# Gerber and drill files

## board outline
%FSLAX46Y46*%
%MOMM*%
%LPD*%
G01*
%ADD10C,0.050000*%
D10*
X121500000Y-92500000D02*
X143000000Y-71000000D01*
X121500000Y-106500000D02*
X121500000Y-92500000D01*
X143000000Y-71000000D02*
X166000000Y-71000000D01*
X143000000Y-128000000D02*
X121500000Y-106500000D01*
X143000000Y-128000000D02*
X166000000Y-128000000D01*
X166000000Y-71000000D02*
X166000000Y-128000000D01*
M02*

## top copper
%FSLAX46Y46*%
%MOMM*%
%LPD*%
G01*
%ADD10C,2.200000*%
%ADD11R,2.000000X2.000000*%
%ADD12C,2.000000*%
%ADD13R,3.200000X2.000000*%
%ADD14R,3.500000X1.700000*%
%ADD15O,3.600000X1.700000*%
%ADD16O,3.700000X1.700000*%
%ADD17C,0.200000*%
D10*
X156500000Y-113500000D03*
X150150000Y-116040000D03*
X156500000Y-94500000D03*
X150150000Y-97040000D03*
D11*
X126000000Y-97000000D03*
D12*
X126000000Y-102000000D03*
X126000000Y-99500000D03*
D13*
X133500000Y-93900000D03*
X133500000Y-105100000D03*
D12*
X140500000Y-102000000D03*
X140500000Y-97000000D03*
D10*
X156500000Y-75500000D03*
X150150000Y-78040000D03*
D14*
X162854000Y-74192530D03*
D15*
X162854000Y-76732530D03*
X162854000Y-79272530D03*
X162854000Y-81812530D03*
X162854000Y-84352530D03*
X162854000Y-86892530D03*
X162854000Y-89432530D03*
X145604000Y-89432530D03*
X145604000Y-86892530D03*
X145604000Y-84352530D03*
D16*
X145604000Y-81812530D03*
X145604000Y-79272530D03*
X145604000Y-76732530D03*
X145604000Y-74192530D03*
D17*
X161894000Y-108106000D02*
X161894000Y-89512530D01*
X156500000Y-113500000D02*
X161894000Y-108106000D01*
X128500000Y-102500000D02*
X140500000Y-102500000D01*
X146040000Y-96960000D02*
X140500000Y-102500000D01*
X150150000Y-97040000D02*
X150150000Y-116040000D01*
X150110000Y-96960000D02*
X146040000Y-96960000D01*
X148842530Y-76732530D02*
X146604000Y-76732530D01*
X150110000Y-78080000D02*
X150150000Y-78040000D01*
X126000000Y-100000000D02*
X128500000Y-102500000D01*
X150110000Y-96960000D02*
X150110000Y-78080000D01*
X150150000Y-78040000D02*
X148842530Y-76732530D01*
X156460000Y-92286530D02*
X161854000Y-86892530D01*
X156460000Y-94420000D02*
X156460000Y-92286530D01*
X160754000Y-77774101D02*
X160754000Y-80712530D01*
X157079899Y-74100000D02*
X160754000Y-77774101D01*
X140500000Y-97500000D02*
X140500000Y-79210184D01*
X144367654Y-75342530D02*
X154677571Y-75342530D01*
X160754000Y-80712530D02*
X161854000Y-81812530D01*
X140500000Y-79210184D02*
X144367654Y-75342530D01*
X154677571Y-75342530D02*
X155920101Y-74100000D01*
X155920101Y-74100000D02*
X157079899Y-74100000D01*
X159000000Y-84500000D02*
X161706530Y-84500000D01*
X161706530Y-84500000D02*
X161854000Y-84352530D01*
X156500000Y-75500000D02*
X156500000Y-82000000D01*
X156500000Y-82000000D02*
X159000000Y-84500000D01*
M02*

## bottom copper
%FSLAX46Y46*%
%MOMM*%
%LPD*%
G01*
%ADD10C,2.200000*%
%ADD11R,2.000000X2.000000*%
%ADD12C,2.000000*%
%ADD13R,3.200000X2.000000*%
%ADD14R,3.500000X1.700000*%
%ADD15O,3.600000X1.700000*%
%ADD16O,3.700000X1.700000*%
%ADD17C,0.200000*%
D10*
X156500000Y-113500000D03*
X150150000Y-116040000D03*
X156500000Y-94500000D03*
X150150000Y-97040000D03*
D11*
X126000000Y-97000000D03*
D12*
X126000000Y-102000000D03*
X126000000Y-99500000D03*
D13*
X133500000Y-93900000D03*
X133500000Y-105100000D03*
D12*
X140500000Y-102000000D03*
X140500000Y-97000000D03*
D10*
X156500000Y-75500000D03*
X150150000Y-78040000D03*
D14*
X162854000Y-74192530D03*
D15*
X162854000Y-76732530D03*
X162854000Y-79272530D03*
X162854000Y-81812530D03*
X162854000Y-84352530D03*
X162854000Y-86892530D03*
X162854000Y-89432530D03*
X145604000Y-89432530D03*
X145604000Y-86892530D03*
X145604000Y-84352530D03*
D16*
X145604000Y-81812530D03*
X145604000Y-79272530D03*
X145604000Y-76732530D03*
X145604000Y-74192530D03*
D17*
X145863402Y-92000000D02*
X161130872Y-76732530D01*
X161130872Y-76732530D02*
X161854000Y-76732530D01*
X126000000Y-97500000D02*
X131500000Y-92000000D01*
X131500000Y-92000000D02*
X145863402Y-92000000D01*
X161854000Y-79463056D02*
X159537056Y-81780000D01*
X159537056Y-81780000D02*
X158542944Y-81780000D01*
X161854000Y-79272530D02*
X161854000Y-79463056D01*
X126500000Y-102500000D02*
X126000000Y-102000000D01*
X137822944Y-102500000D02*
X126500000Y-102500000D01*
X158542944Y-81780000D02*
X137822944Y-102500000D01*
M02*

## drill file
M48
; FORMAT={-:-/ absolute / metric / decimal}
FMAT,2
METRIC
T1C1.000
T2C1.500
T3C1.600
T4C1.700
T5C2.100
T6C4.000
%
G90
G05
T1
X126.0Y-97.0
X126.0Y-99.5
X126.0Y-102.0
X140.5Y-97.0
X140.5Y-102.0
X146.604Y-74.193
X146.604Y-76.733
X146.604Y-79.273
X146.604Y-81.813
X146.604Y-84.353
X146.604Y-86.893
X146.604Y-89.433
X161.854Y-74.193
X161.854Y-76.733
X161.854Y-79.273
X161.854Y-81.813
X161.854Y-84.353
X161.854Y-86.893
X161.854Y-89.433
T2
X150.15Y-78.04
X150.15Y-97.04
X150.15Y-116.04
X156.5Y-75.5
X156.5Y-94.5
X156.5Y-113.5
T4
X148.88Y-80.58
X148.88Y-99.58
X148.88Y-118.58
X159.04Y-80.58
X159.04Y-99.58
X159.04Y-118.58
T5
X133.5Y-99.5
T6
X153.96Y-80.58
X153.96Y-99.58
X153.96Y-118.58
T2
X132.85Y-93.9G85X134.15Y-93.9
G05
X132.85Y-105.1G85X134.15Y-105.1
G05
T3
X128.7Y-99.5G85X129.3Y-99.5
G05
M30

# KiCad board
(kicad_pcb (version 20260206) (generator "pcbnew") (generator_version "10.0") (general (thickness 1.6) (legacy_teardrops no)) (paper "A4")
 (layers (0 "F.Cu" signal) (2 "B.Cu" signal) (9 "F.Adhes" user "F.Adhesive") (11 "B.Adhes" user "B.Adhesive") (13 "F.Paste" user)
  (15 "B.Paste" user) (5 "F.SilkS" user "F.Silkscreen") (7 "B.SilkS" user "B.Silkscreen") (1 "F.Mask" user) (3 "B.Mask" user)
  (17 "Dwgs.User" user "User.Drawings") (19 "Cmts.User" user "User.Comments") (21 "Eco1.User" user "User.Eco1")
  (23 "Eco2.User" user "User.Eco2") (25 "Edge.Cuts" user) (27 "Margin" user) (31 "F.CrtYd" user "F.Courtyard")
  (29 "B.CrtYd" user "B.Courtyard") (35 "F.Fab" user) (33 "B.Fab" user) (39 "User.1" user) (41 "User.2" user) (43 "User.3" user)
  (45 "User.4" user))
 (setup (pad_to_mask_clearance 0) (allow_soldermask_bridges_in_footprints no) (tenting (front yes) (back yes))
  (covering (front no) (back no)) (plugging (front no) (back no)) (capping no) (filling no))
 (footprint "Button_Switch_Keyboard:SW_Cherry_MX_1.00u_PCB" (layer "F.Cu") (at 156.5 113.5)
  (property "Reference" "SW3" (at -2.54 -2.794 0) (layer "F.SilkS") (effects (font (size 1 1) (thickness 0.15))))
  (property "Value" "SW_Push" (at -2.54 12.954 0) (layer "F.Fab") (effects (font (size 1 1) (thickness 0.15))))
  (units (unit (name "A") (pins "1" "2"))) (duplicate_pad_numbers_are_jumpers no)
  (pad "" np_thru_hole circle (at -7.62 5.08) (size 1.7 1.7) (drill 1.7) (layers "*.Cu" "*.Mask"))
  (pad "" np_thru_hole circle (at -2.54 5.08) (size 4 4) (drill 4) (layers "*.Cu" "*.Mask"))
  (pad "" np_thru_hole circle (at 2.54 5.08) (size 1.7 1.7) (drill 1.7) (layers "*.Cu" "*.Mask"))
  (pad "1" thru_hole circle (at 0 0) (size 2.2 2.2) (drill 1.5) (layers "*.Cu" "*.Mask") (remove_unused_layers no)
   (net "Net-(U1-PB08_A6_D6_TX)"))
  (pad "2" thru_hole circle (at -6.35 2.54) (size 2.2 2.2) (drill 1.5) (layers "*.Cu" "*.Mask") (remove_unused_layers no) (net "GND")))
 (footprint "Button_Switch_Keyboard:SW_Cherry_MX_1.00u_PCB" (layer "F.Cu") (at 156.5 94.5)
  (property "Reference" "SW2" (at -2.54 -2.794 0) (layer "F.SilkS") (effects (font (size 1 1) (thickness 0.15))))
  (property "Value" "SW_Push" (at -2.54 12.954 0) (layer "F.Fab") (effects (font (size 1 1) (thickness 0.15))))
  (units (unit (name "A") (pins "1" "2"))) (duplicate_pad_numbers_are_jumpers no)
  (pad "" np_thru_hole circle (at -7.62 5.08) (size 1.7 1.7) (drill 1.7) (layers "*.Cu" "*.Mask"))
  (pad "" np_thru_hole circle (at -2.54 5.08) (size 4 4) (drill 4) (layers "*.Cu" "*.Mask"))
  (pad "" np_thru_hole circle (at 2.54 5.08) (size 1.7 1.7) (drill 1.7) (layers "*.Cu" "*.Mask"))
  (pad "1" thru_hole circle (at 0 0) (size 2.2 2.2) (drill 1.5) (layers "*.Cu" "*.Mask") (remove_unused_layers no)
   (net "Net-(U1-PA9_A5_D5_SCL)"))
  (pad "2" thru_hole circle (at -6.35 2.54) (size 2.2 2.2) (drill 1.5) (layers "*.Cu" "*.Mask") (remove_unused_layers no) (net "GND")))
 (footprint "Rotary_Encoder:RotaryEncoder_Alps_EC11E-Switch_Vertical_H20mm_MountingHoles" (layer "F.Cu") (at 126 97)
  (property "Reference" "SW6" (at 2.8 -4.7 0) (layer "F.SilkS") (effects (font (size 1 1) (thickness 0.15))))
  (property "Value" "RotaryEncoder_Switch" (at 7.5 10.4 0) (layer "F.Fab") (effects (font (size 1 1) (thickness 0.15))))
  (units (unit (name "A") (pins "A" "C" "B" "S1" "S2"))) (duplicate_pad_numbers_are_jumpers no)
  (pad "" np_thru_hole oval (at 3 2.5) (size 2.2 1.6) (drill oval 2.2 1.6) (layers "*.Mask"))
  (pad "" np_thru_hole circle (at 7.5 2.5) (size 2.1 2.1) (drill 2.1) (layers "*.Mask"))
  (pad "A" thru_hole rect (at 0 0) (size 2 2) (drill 1) (layers "*.Cu" "*.Mask") (remove_unused_layers no) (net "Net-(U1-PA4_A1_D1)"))
  (pad "B" thru_hole circle (at 0 5) (size 2 2) (drill 1) (layers "*.Cu" "*.Mask") (remove_unused_layers no) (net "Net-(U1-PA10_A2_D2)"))
  (pad "C" thru_hole circle (at 0 2.5) (size 2 2) (drill 1) (layers "*.Cu" "*.Mask") (remove_unused_layers no) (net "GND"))
  (pad "MP" thru_hole rect (at 7.5 -3.1) (size 3.2 2) (drill oval 2.8 1.5) (layers "*.Cu" "*.Mask") (remove_unused_layers no))
  (pad "MP" thru_hole rect (at 7.5 8.1) (size 3.2 2) (drill oval 2.8 1.5) (layers "*.Cu" "*.Mask") (remove_unused_layers no))
  (pad "S1" thru_hole circle (at 14.5 5) (size 2 2) (drill 1) (layers "*.Cu" "*.Mask") (remove_unused_layers no) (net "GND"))
  (pad "S2" thru_hole circle (at 14.5 0) (size 2 2) (drill 1) (layers "*.Cu" "*.Mask") (remove_unused_layers no) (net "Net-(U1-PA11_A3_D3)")))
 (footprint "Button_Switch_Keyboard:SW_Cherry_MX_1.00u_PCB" (layer "F.Cu") (at 156.5 75.5)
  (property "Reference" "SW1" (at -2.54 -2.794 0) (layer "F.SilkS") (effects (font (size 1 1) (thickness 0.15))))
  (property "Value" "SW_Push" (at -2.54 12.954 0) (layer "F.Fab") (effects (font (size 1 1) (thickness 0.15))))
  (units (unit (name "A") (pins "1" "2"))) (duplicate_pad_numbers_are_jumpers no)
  (pad "" np_thru_hole circle (at -7.62 5.08) (size 1.7 1.7) (drill 1.7) (layers "*.Cu" "*.Mask"))
  (pad "" np_thru_hole circle (at -2.54 5.08) (size 4 4) (drill 4) (layers "*.Cu" "*.Mask"))
  (pad "" np_thru_hole circle (at 2.54 5.08) (size 1.7 1.7) (drill 1.7) (layers "*.Cu" "*.Mask"))
  (pad "1" thru_hole circle (at 0 0) (size 2.2 2.2) (drill 1.5) (layers "*.Cu" "*.Mask") (remove_unused_layers no)
   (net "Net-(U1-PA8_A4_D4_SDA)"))
  (pad "2" thru_hole circle (at -6.35 2.54) (size 2.2 2.2) (drill 1.5) (layers "*.Cu" "*.Mask") (remove_unused_layers no) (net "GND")))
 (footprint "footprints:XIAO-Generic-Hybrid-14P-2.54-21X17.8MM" (layer "B.Cu") (at 154.229 81.81253 180)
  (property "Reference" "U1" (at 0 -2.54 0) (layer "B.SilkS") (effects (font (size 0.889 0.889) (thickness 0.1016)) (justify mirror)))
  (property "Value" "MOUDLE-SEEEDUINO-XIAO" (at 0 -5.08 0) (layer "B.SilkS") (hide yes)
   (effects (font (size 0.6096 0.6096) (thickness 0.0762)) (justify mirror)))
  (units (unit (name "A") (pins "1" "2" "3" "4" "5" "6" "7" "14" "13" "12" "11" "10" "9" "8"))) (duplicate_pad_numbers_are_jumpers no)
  (pad "1" thru_hole rect (at -7.625 7.62 180) (size 3.5 1.7) (drill 1 (offset -1 0)) (layers "*.Cu" "*.Mask") (remove_unused_layers no)
   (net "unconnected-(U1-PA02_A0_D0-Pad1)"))
  (pad "2" thru_hole oval (at -7.625 5.08 180) (size 3.6 1.7) (drill 1 (offset -1 0)) (layers "*.Cu" "*.Mask") (remove_unused_layers no)
   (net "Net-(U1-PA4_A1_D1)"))
  (pad "3" thru_hole oval (at -7.625 2.54 180) (size 3.6 1.7) (drill 1 (offset -1 0)) (layers "*.Cu" "*.Mask") (remove_unused_layers no)
   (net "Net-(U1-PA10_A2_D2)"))
  (pad "4" thru_hole oval (at -7.625 0 180) (size 3.6 1.7) (drill 1 (offset -1 0)) (layers "*.Cu" "*.Mask") (remove_unused_layers no)
   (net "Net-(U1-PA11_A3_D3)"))
  (pad "5" thru_hole oval (at -7.625 -2.54 180) (size 3.6 1.7) (drill 1 (offset -1 0)) (layers "*.Cu" "*.Mask") (remove_unused_layers no)
   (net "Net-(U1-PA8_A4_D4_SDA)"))
  (pad "6" thru_hole oval (at -7.625 -5.08) (size 3.6 1.7) (drill 1 (offset 1 0)) (layers "*.Cu" "*.Mask") (remove_unused_layers no)
   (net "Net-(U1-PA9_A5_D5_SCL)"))
  (pad "7" thru_hole oval (at -7.625 -7.62 180) (size 3.6 1.7) (drill 1 (offset -1 0)) (layers "*.Cu" "*.Mask") (remove_unused_layers no)
   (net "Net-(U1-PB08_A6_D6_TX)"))
  (pad "8" thru_hole oval (at 7.625 -7.62 180) (size 3.6 1.7) (drill 1 (offset 1 0)) (layers "*.Cu" "*.Mask") (remove_unused_layers no)
   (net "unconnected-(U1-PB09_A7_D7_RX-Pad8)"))
  (pad "9" thru_hole oval (at 7.625 -5.08 180) (size 3.6 1.7) (drill 1 (offset 1 0)) (layers "*.Cu" "*.Mask") (remove_unused_layers no)
   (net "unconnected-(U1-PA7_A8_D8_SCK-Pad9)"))
  (pad "10" thru_hole oval (at 7.625 -2.54 180) (size 3.6 1.7) (drill 1 (offset 1 0)) (layers "*.Cu" "*.Mask") (remove_unused_layers no)
   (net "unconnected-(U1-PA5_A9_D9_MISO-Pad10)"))
  (pad "11" thru_hole oval (at 7.625 0 180) (size 3.7 1.7) (drill 1 (offset 1 0)) (layers "*.Cu" "*.Mask") (remove_unused_layers no)
   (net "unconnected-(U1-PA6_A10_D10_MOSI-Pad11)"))
  (pad "12" thru_hole oval (at 7.625 2.54 180) (size 3.7 1.7) (drill 1 (offset 1 0)) (layers "*.Cu" "*.Mask") (remove_unused_layers no)
   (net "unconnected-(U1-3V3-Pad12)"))
  (pad "13" thru_hole oval (at 7.625 5.08 180) (size 3.7 1.7) (drill 1 (offset 1 0)) (layers "*.Cu" "*.Mask") (remove_unused_layers no)
   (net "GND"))
  (pad "14" thru_hole oval (at 7.625 7.62 180) (size 3.7 1.7) (drill 1 (offset 1 0)) (layers "*.Cu" "*.Mask") (remove_unused_layers no)
   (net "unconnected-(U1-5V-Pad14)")))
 (gr_line (start 121.5 92.5) (end 143 71) (stroke (width 0.05) (type default)) (layer "Edge.Cuts"))
 (gr_line (start 121.5 106.5) (end 121.5 92.5) (stroke (width 0.05) (type default)) (layer "Edge.Cuts"))
 (gr_line (start 143 71) (end 166 71) (stroke (width 0.05) (type default)) (layer "Edge.Cuts"))
 (gr_line (start 143 128) (end 121.5 106.5) (stroke (width 0.05) (type default)) (layer "Edge.Cuts"))
 (gr_line (start 143 128) (end 166 128) (stroke (width 0.05) (type default)) (layer "Edge.Cuts"))
 (gr_line (start 166 71) (end 166 128) (stroke (width 0.05) (type default)) (layer "Edge.Cuts"))
 (segment (start 161.894 108.106) (end 161.894 89.51253) (width 0.2) (layer "F.Cu") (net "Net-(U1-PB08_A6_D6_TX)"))
 (segment (start 156.5 113.5) (end 161.894 108.106) (width 0.2) (layer "F.Cu") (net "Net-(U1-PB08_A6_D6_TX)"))
 (segment (start 128.5 102.5) (end 140.5 102.5) (width 0.2) (layer "F.Cu") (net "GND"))
 (segment (start 146.04 96.96) (end 140.5 102.5) (width 0.2) (layer "F.Cu") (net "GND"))
 (segment (start 150.15 97.04) (end 150.15 116.04) (width 0.2) (layer "F.Cu") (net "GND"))
 (segment (start 150.11 96.96) (end 146.04 96.96) (width 0.2) (layer "F.Cu") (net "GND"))
 (segment (start 148.84253 76.73253) (end 146.604 76.73253) (width 0.2) (layer "F.Cu") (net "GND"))
 (segment (start 150.11 78.08) (end 150.15 78.04) (width 0.2) (layer "F.Cu") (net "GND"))
 (segment (start 126 100) (end 128.5 102.5) (width 0.2) (layer "F.Cu") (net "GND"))
 (segment (start 150.11 96.96) (end 150.11 78.08) (width 0.2) (layer "F.Cu") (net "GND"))
 (segment (start 150.15 78.04) (end 148.84253 76.73253) (width 0.2) (layer "F.Cu") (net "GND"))
 (segment (start 156.46 92.28653) (end 161.854 86.89253) (width 0.2) (layer "F.Cu") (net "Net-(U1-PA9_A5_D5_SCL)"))
 (segment (start 156.46 94.42) (end 156.46 92.28653) (width 0.2) (layer "F.Cu") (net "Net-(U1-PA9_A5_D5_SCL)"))
 (segment (start 145.863402 92) (end 161.130872 76.73253) (width 0.2) (layer "B.Cu") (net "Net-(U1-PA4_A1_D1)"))
 (segment (start 161.130872 76.73253) (end 161.854 76.73253) (width 0.2) (layer "B.Cu") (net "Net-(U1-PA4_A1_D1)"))
 (segment (start 126 97.5) (end 131.5 92) (width 0.2) (layer "B.Cu") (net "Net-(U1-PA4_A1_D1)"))
 (segment (start 131.5 92) (end 145.863402 92) (width 0.2) (layer "B.Cu") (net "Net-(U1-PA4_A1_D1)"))
 (segment (start 161.854 79.463056) (end 159.537056 81.78) (width 0.2) (layer "B.Cu") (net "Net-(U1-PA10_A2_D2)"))
 (segment (start 159.537056 81.78) (end 158.542944 81.78) (width 0.2) (layer "B.Cu") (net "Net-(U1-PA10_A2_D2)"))
 (segment (start 161.854 79.27253) (end 161.854 79.463056) (width 0.2) (layer "B.Cu") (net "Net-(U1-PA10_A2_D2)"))
 (segment (start 126.5 102.5) (end 126 102) (width 0.2) (layer "B.Cu") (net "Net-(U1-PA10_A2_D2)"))
 (segment (start 137.822944 102.5) (end 126.5 102.5) (width 0.2) (layer "B.Cu") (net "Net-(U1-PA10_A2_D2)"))
 (segment (start 158.542944 81.78) (end 137.822944 102.5) (width 0.2) (layer "B.Cu") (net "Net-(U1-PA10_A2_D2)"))
 (segment (start 160.754 77.774101) (end 160.754 80.71253) (width 0.2) (layer "F.Cu") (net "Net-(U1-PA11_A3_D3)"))
 (segment (start 157.079899 74.1) (end 160.754 77.774101) (width 0.2) (layer "F.Cu") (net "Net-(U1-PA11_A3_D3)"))
 (segment (start 140.5 97.5) (end 140.5 79.210184) (width 0.2) (layer "F.Cu") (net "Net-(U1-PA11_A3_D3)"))
 (segment (start 144.367654 75.34253) (end 154.677571 75.34253) (width 0.2) (layer "F.Cu") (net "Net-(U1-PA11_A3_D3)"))
 (segment (start 160.754 80.71253) (end 161.854 81.81253) (width 0.2) (layer "F.Cu") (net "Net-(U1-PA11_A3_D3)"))
 (segment (start 140.5 79.210184) (end 144.367654 75.34253) (width 0.2) (layer "F.Cu") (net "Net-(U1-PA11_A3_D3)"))
 (segment (start 154.677571 75.34253) (end 155.920101 74.1) (width 0.2) (layer "F.Cu") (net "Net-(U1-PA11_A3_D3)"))
 (segment (start 155.920101 74.1) (end 157.079899 74.1) (width 0.2) (layer "F.Cu") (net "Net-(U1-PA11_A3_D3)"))
 (segment (start 159 84.5) (end 161.70653 84.5) (width 0.2) (layer "F.Cu") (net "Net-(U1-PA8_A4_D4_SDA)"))
 (segment (start 161.70653 84.5) (end 161.854 84.35253) (width 0.2) (layer "F.Cu") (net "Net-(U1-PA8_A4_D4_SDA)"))
 (segment (start 156.5 75.5) (end 156.5 82) (width 0.2) (layer "F.Cu") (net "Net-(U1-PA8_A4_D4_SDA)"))
 (segment (start 156.5 82) (end 159 84.5) (width 0.2) (layer "F.Cu") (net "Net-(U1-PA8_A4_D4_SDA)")))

